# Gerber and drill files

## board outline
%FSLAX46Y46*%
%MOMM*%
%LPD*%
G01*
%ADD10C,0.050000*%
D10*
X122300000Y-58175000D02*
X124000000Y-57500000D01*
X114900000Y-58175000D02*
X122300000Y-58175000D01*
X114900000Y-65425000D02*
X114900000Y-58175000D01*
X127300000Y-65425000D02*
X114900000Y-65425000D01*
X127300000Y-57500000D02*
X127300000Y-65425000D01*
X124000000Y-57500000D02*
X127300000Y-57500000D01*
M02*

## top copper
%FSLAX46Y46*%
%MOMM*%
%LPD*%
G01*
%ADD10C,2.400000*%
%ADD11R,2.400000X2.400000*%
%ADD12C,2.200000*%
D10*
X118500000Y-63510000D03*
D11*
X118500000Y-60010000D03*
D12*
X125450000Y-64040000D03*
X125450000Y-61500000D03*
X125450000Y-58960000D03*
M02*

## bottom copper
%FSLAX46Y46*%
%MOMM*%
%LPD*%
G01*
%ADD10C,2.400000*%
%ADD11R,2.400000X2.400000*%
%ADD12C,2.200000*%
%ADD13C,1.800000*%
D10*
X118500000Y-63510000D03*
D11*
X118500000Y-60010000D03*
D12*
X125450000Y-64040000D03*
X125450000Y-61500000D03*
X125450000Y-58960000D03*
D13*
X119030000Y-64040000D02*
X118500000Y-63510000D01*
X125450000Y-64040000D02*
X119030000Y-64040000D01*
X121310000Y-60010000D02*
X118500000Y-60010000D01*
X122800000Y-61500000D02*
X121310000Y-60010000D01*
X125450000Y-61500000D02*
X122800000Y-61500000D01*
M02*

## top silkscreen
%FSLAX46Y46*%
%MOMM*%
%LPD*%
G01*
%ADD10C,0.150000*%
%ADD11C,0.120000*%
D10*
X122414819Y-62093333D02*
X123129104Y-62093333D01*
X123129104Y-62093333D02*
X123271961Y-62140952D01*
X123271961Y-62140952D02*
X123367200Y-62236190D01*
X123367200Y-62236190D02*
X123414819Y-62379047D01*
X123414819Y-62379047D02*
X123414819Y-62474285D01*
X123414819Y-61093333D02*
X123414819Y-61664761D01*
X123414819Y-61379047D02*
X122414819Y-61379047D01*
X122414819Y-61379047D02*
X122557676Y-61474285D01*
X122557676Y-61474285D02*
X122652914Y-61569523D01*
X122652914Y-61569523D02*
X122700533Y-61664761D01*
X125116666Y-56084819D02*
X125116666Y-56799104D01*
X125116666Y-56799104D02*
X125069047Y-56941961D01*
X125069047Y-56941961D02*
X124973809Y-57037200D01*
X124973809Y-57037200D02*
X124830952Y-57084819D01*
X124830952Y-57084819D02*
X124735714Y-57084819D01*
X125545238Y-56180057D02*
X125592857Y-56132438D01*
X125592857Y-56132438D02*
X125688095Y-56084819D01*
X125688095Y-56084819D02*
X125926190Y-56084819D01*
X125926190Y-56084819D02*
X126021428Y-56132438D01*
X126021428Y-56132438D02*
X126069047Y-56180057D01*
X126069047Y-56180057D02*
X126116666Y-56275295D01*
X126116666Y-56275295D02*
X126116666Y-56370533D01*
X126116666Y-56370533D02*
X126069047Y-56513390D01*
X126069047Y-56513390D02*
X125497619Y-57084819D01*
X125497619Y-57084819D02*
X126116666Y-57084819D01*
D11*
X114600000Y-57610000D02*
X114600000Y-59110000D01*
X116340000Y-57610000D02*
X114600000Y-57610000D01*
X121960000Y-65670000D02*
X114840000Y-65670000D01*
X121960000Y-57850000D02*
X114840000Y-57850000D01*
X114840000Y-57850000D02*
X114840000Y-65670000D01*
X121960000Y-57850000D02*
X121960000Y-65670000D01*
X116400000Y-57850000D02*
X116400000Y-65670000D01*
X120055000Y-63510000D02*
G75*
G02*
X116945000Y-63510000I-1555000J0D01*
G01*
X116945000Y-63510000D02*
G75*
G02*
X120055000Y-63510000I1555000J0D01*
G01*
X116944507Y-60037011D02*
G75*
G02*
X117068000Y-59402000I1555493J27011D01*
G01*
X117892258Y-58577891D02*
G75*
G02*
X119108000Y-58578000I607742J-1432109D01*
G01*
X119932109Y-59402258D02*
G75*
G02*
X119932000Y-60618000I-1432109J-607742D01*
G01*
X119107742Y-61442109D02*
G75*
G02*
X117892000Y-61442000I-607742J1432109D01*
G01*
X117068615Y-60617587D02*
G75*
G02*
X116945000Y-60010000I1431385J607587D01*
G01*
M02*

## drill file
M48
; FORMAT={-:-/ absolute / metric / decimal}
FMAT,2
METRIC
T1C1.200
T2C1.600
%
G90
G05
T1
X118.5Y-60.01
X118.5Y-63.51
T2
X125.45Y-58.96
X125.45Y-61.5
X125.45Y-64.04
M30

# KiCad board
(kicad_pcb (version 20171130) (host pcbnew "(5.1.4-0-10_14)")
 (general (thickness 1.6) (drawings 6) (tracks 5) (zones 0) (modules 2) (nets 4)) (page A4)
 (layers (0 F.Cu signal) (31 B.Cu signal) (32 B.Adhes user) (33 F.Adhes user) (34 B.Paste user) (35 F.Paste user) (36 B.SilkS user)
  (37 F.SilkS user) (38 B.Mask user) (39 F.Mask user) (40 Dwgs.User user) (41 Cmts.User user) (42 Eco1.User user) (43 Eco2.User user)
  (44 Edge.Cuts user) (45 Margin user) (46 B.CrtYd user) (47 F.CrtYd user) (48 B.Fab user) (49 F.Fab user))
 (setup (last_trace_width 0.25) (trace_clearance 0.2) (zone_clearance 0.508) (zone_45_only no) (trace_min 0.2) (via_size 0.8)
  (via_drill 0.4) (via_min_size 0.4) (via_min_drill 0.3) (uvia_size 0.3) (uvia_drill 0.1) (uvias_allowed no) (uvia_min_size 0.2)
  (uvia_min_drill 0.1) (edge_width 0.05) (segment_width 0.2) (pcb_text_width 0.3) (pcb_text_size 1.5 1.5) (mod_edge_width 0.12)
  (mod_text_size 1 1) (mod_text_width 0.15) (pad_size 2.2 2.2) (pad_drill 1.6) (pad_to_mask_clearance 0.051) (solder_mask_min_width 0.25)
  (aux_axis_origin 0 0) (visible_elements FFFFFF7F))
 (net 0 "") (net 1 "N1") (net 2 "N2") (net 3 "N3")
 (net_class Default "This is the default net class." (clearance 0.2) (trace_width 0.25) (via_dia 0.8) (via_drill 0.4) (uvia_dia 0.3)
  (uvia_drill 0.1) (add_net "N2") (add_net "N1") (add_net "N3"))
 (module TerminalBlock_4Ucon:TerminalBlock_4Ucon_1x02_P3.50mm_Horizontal (layer F.Cu) (at 118.5 60.01 270)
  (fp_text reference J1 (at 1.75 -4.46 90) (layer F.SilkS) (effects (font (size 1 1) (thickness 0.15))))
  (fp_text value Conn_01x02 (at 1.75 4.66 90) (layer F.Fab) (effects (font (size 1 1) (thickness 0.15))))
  (fp_line (start -2.4 3.9) (end -0.9 3.9) (layer F.SilkS) (width 0.12))
  (fp_line (start -2.4 2.16) (end -2.4 3.9) (layer F.SilkS) (width 0.12))
  (fp_line (start 5.66 -3.46) (end 5.66 3.66) (layer F.SilkS) (width 0.12))
  (fp_line (start -2.16 -3.46) (end -2.16 3.66) (layer F.SilkS) (width 0.12))
  (fp_line (start -2.16 3.66) (end 5.66 3.66) (layer F.SilkS) (width 0.12))
  (fp_line (start -2.16 -3.46) (end 5.66 -3.46) (layer F.SilkS) (width 0.12))
  (fp_line (start -2.16 2.1) (end 5.66 2.1) (layer F.SilkS) (width 0.12))
  (fp_circle (center 3.5 0) (end 5.055 0) (layer F.SilkS) (width 0.12))
  (fp_arc (start 0 0) (end -0.608 1.432) (angle -24) (layer F.SilkS) (width 0.12))
  (fp_arc (start 0 0) (end -1.432 -0.608) (angle -46) (layer F.SilkS) (width 0.12))
  (fp_arc (start 0 0) (end 0.608 -1.432) (angle -46) (layer F.SilkS) (width 0.12))
  (fp_arc (start 0 0) (end 1.432 0.608) (angle -46) (layer F.SilkS) (width 0.12))
  (fp_arc (start 0 0) (end 0 1.555) (angle -23) (layer F.SilkS) (width 0.12))
  (pad 2 thru_hole circle (at 3.5 0 270) (size 2.4 2.4) (drill 1.2) (layers *.Cu *.Mask) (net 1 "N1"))
  (pad 1 thru_hole rect (at 0 0 270) (size 2.4 2.4) (drill 1.2) (layers *.Cu *.Mask) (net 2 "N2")))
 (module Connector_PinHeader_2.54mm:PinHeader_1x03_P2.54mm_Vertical (layer F.Cu) (at 125.45 58.96)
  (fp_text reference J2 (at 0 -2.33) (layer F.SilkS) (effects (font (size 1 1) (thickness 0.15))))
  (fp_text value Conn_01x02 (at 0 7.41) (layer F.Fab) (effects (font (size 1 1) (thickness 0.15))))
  (pad 3 thru_hole circle (at 0 5.08) (size 2.2 2.2) (drill 1.6) (layers *.Cu *.Mask) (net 1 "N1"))
  (pad 2 thru_hole circle (at 0 2.54) (size 2.2 2.2) (drill 1.6) (layers *.Cu *.Mask) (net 2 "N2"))
  (pad 1 thru_hole circle (at 0 0) (size 2.2 2.2) (drill 1.6) (layers *.Cu *.Mask) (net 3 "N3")))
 (gr_line (start 122.3 58.175) (end 124 57.5) (layer Edge.Cuts) (width 0.05))
 (gr_line (start 114.9 58.175) (end 122.3 58.175) (layer Edge.Cuts) (width 0.05))
 (gr_line (start 114.9 65.425) (end 114.9 58.175) (layer Edge.Cuts) (width 0.05))
 (gr_line (start 127.3 65.425) (end 114.9 65.425) (layer Edge.Cuts) (width 0.05))
 (gr_line (start 127.3 57.5) (end 127.3 65.425) (layer Edge.Cuts) (width 0.05))
 (gr_line (start 124 57.5) (end 127.3 57.5) (layer Edge.Cuts) (width 0.05))
 (segment (start 119.03 64.04) (end 118.5 63.51) (width 1.8) (layer B.Cu) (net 1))
 (segment (start 125.45 64.04) (end 119.03 64.04) (width 1.8) (layer B.Cu) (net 1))
 (segment (start 121.31 60.01) (end 118.5 60.01) (width 1.8) (layer B.Cu) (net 2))
 (segment (start 122.8 61.5) (end 121.31 60.01) (width 1.8) (layer B.Cu) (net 2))
 (segment (start 125.45 61.5) (end 122.8 61.5) (width 1.8) (layer B.Cu) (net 2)))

